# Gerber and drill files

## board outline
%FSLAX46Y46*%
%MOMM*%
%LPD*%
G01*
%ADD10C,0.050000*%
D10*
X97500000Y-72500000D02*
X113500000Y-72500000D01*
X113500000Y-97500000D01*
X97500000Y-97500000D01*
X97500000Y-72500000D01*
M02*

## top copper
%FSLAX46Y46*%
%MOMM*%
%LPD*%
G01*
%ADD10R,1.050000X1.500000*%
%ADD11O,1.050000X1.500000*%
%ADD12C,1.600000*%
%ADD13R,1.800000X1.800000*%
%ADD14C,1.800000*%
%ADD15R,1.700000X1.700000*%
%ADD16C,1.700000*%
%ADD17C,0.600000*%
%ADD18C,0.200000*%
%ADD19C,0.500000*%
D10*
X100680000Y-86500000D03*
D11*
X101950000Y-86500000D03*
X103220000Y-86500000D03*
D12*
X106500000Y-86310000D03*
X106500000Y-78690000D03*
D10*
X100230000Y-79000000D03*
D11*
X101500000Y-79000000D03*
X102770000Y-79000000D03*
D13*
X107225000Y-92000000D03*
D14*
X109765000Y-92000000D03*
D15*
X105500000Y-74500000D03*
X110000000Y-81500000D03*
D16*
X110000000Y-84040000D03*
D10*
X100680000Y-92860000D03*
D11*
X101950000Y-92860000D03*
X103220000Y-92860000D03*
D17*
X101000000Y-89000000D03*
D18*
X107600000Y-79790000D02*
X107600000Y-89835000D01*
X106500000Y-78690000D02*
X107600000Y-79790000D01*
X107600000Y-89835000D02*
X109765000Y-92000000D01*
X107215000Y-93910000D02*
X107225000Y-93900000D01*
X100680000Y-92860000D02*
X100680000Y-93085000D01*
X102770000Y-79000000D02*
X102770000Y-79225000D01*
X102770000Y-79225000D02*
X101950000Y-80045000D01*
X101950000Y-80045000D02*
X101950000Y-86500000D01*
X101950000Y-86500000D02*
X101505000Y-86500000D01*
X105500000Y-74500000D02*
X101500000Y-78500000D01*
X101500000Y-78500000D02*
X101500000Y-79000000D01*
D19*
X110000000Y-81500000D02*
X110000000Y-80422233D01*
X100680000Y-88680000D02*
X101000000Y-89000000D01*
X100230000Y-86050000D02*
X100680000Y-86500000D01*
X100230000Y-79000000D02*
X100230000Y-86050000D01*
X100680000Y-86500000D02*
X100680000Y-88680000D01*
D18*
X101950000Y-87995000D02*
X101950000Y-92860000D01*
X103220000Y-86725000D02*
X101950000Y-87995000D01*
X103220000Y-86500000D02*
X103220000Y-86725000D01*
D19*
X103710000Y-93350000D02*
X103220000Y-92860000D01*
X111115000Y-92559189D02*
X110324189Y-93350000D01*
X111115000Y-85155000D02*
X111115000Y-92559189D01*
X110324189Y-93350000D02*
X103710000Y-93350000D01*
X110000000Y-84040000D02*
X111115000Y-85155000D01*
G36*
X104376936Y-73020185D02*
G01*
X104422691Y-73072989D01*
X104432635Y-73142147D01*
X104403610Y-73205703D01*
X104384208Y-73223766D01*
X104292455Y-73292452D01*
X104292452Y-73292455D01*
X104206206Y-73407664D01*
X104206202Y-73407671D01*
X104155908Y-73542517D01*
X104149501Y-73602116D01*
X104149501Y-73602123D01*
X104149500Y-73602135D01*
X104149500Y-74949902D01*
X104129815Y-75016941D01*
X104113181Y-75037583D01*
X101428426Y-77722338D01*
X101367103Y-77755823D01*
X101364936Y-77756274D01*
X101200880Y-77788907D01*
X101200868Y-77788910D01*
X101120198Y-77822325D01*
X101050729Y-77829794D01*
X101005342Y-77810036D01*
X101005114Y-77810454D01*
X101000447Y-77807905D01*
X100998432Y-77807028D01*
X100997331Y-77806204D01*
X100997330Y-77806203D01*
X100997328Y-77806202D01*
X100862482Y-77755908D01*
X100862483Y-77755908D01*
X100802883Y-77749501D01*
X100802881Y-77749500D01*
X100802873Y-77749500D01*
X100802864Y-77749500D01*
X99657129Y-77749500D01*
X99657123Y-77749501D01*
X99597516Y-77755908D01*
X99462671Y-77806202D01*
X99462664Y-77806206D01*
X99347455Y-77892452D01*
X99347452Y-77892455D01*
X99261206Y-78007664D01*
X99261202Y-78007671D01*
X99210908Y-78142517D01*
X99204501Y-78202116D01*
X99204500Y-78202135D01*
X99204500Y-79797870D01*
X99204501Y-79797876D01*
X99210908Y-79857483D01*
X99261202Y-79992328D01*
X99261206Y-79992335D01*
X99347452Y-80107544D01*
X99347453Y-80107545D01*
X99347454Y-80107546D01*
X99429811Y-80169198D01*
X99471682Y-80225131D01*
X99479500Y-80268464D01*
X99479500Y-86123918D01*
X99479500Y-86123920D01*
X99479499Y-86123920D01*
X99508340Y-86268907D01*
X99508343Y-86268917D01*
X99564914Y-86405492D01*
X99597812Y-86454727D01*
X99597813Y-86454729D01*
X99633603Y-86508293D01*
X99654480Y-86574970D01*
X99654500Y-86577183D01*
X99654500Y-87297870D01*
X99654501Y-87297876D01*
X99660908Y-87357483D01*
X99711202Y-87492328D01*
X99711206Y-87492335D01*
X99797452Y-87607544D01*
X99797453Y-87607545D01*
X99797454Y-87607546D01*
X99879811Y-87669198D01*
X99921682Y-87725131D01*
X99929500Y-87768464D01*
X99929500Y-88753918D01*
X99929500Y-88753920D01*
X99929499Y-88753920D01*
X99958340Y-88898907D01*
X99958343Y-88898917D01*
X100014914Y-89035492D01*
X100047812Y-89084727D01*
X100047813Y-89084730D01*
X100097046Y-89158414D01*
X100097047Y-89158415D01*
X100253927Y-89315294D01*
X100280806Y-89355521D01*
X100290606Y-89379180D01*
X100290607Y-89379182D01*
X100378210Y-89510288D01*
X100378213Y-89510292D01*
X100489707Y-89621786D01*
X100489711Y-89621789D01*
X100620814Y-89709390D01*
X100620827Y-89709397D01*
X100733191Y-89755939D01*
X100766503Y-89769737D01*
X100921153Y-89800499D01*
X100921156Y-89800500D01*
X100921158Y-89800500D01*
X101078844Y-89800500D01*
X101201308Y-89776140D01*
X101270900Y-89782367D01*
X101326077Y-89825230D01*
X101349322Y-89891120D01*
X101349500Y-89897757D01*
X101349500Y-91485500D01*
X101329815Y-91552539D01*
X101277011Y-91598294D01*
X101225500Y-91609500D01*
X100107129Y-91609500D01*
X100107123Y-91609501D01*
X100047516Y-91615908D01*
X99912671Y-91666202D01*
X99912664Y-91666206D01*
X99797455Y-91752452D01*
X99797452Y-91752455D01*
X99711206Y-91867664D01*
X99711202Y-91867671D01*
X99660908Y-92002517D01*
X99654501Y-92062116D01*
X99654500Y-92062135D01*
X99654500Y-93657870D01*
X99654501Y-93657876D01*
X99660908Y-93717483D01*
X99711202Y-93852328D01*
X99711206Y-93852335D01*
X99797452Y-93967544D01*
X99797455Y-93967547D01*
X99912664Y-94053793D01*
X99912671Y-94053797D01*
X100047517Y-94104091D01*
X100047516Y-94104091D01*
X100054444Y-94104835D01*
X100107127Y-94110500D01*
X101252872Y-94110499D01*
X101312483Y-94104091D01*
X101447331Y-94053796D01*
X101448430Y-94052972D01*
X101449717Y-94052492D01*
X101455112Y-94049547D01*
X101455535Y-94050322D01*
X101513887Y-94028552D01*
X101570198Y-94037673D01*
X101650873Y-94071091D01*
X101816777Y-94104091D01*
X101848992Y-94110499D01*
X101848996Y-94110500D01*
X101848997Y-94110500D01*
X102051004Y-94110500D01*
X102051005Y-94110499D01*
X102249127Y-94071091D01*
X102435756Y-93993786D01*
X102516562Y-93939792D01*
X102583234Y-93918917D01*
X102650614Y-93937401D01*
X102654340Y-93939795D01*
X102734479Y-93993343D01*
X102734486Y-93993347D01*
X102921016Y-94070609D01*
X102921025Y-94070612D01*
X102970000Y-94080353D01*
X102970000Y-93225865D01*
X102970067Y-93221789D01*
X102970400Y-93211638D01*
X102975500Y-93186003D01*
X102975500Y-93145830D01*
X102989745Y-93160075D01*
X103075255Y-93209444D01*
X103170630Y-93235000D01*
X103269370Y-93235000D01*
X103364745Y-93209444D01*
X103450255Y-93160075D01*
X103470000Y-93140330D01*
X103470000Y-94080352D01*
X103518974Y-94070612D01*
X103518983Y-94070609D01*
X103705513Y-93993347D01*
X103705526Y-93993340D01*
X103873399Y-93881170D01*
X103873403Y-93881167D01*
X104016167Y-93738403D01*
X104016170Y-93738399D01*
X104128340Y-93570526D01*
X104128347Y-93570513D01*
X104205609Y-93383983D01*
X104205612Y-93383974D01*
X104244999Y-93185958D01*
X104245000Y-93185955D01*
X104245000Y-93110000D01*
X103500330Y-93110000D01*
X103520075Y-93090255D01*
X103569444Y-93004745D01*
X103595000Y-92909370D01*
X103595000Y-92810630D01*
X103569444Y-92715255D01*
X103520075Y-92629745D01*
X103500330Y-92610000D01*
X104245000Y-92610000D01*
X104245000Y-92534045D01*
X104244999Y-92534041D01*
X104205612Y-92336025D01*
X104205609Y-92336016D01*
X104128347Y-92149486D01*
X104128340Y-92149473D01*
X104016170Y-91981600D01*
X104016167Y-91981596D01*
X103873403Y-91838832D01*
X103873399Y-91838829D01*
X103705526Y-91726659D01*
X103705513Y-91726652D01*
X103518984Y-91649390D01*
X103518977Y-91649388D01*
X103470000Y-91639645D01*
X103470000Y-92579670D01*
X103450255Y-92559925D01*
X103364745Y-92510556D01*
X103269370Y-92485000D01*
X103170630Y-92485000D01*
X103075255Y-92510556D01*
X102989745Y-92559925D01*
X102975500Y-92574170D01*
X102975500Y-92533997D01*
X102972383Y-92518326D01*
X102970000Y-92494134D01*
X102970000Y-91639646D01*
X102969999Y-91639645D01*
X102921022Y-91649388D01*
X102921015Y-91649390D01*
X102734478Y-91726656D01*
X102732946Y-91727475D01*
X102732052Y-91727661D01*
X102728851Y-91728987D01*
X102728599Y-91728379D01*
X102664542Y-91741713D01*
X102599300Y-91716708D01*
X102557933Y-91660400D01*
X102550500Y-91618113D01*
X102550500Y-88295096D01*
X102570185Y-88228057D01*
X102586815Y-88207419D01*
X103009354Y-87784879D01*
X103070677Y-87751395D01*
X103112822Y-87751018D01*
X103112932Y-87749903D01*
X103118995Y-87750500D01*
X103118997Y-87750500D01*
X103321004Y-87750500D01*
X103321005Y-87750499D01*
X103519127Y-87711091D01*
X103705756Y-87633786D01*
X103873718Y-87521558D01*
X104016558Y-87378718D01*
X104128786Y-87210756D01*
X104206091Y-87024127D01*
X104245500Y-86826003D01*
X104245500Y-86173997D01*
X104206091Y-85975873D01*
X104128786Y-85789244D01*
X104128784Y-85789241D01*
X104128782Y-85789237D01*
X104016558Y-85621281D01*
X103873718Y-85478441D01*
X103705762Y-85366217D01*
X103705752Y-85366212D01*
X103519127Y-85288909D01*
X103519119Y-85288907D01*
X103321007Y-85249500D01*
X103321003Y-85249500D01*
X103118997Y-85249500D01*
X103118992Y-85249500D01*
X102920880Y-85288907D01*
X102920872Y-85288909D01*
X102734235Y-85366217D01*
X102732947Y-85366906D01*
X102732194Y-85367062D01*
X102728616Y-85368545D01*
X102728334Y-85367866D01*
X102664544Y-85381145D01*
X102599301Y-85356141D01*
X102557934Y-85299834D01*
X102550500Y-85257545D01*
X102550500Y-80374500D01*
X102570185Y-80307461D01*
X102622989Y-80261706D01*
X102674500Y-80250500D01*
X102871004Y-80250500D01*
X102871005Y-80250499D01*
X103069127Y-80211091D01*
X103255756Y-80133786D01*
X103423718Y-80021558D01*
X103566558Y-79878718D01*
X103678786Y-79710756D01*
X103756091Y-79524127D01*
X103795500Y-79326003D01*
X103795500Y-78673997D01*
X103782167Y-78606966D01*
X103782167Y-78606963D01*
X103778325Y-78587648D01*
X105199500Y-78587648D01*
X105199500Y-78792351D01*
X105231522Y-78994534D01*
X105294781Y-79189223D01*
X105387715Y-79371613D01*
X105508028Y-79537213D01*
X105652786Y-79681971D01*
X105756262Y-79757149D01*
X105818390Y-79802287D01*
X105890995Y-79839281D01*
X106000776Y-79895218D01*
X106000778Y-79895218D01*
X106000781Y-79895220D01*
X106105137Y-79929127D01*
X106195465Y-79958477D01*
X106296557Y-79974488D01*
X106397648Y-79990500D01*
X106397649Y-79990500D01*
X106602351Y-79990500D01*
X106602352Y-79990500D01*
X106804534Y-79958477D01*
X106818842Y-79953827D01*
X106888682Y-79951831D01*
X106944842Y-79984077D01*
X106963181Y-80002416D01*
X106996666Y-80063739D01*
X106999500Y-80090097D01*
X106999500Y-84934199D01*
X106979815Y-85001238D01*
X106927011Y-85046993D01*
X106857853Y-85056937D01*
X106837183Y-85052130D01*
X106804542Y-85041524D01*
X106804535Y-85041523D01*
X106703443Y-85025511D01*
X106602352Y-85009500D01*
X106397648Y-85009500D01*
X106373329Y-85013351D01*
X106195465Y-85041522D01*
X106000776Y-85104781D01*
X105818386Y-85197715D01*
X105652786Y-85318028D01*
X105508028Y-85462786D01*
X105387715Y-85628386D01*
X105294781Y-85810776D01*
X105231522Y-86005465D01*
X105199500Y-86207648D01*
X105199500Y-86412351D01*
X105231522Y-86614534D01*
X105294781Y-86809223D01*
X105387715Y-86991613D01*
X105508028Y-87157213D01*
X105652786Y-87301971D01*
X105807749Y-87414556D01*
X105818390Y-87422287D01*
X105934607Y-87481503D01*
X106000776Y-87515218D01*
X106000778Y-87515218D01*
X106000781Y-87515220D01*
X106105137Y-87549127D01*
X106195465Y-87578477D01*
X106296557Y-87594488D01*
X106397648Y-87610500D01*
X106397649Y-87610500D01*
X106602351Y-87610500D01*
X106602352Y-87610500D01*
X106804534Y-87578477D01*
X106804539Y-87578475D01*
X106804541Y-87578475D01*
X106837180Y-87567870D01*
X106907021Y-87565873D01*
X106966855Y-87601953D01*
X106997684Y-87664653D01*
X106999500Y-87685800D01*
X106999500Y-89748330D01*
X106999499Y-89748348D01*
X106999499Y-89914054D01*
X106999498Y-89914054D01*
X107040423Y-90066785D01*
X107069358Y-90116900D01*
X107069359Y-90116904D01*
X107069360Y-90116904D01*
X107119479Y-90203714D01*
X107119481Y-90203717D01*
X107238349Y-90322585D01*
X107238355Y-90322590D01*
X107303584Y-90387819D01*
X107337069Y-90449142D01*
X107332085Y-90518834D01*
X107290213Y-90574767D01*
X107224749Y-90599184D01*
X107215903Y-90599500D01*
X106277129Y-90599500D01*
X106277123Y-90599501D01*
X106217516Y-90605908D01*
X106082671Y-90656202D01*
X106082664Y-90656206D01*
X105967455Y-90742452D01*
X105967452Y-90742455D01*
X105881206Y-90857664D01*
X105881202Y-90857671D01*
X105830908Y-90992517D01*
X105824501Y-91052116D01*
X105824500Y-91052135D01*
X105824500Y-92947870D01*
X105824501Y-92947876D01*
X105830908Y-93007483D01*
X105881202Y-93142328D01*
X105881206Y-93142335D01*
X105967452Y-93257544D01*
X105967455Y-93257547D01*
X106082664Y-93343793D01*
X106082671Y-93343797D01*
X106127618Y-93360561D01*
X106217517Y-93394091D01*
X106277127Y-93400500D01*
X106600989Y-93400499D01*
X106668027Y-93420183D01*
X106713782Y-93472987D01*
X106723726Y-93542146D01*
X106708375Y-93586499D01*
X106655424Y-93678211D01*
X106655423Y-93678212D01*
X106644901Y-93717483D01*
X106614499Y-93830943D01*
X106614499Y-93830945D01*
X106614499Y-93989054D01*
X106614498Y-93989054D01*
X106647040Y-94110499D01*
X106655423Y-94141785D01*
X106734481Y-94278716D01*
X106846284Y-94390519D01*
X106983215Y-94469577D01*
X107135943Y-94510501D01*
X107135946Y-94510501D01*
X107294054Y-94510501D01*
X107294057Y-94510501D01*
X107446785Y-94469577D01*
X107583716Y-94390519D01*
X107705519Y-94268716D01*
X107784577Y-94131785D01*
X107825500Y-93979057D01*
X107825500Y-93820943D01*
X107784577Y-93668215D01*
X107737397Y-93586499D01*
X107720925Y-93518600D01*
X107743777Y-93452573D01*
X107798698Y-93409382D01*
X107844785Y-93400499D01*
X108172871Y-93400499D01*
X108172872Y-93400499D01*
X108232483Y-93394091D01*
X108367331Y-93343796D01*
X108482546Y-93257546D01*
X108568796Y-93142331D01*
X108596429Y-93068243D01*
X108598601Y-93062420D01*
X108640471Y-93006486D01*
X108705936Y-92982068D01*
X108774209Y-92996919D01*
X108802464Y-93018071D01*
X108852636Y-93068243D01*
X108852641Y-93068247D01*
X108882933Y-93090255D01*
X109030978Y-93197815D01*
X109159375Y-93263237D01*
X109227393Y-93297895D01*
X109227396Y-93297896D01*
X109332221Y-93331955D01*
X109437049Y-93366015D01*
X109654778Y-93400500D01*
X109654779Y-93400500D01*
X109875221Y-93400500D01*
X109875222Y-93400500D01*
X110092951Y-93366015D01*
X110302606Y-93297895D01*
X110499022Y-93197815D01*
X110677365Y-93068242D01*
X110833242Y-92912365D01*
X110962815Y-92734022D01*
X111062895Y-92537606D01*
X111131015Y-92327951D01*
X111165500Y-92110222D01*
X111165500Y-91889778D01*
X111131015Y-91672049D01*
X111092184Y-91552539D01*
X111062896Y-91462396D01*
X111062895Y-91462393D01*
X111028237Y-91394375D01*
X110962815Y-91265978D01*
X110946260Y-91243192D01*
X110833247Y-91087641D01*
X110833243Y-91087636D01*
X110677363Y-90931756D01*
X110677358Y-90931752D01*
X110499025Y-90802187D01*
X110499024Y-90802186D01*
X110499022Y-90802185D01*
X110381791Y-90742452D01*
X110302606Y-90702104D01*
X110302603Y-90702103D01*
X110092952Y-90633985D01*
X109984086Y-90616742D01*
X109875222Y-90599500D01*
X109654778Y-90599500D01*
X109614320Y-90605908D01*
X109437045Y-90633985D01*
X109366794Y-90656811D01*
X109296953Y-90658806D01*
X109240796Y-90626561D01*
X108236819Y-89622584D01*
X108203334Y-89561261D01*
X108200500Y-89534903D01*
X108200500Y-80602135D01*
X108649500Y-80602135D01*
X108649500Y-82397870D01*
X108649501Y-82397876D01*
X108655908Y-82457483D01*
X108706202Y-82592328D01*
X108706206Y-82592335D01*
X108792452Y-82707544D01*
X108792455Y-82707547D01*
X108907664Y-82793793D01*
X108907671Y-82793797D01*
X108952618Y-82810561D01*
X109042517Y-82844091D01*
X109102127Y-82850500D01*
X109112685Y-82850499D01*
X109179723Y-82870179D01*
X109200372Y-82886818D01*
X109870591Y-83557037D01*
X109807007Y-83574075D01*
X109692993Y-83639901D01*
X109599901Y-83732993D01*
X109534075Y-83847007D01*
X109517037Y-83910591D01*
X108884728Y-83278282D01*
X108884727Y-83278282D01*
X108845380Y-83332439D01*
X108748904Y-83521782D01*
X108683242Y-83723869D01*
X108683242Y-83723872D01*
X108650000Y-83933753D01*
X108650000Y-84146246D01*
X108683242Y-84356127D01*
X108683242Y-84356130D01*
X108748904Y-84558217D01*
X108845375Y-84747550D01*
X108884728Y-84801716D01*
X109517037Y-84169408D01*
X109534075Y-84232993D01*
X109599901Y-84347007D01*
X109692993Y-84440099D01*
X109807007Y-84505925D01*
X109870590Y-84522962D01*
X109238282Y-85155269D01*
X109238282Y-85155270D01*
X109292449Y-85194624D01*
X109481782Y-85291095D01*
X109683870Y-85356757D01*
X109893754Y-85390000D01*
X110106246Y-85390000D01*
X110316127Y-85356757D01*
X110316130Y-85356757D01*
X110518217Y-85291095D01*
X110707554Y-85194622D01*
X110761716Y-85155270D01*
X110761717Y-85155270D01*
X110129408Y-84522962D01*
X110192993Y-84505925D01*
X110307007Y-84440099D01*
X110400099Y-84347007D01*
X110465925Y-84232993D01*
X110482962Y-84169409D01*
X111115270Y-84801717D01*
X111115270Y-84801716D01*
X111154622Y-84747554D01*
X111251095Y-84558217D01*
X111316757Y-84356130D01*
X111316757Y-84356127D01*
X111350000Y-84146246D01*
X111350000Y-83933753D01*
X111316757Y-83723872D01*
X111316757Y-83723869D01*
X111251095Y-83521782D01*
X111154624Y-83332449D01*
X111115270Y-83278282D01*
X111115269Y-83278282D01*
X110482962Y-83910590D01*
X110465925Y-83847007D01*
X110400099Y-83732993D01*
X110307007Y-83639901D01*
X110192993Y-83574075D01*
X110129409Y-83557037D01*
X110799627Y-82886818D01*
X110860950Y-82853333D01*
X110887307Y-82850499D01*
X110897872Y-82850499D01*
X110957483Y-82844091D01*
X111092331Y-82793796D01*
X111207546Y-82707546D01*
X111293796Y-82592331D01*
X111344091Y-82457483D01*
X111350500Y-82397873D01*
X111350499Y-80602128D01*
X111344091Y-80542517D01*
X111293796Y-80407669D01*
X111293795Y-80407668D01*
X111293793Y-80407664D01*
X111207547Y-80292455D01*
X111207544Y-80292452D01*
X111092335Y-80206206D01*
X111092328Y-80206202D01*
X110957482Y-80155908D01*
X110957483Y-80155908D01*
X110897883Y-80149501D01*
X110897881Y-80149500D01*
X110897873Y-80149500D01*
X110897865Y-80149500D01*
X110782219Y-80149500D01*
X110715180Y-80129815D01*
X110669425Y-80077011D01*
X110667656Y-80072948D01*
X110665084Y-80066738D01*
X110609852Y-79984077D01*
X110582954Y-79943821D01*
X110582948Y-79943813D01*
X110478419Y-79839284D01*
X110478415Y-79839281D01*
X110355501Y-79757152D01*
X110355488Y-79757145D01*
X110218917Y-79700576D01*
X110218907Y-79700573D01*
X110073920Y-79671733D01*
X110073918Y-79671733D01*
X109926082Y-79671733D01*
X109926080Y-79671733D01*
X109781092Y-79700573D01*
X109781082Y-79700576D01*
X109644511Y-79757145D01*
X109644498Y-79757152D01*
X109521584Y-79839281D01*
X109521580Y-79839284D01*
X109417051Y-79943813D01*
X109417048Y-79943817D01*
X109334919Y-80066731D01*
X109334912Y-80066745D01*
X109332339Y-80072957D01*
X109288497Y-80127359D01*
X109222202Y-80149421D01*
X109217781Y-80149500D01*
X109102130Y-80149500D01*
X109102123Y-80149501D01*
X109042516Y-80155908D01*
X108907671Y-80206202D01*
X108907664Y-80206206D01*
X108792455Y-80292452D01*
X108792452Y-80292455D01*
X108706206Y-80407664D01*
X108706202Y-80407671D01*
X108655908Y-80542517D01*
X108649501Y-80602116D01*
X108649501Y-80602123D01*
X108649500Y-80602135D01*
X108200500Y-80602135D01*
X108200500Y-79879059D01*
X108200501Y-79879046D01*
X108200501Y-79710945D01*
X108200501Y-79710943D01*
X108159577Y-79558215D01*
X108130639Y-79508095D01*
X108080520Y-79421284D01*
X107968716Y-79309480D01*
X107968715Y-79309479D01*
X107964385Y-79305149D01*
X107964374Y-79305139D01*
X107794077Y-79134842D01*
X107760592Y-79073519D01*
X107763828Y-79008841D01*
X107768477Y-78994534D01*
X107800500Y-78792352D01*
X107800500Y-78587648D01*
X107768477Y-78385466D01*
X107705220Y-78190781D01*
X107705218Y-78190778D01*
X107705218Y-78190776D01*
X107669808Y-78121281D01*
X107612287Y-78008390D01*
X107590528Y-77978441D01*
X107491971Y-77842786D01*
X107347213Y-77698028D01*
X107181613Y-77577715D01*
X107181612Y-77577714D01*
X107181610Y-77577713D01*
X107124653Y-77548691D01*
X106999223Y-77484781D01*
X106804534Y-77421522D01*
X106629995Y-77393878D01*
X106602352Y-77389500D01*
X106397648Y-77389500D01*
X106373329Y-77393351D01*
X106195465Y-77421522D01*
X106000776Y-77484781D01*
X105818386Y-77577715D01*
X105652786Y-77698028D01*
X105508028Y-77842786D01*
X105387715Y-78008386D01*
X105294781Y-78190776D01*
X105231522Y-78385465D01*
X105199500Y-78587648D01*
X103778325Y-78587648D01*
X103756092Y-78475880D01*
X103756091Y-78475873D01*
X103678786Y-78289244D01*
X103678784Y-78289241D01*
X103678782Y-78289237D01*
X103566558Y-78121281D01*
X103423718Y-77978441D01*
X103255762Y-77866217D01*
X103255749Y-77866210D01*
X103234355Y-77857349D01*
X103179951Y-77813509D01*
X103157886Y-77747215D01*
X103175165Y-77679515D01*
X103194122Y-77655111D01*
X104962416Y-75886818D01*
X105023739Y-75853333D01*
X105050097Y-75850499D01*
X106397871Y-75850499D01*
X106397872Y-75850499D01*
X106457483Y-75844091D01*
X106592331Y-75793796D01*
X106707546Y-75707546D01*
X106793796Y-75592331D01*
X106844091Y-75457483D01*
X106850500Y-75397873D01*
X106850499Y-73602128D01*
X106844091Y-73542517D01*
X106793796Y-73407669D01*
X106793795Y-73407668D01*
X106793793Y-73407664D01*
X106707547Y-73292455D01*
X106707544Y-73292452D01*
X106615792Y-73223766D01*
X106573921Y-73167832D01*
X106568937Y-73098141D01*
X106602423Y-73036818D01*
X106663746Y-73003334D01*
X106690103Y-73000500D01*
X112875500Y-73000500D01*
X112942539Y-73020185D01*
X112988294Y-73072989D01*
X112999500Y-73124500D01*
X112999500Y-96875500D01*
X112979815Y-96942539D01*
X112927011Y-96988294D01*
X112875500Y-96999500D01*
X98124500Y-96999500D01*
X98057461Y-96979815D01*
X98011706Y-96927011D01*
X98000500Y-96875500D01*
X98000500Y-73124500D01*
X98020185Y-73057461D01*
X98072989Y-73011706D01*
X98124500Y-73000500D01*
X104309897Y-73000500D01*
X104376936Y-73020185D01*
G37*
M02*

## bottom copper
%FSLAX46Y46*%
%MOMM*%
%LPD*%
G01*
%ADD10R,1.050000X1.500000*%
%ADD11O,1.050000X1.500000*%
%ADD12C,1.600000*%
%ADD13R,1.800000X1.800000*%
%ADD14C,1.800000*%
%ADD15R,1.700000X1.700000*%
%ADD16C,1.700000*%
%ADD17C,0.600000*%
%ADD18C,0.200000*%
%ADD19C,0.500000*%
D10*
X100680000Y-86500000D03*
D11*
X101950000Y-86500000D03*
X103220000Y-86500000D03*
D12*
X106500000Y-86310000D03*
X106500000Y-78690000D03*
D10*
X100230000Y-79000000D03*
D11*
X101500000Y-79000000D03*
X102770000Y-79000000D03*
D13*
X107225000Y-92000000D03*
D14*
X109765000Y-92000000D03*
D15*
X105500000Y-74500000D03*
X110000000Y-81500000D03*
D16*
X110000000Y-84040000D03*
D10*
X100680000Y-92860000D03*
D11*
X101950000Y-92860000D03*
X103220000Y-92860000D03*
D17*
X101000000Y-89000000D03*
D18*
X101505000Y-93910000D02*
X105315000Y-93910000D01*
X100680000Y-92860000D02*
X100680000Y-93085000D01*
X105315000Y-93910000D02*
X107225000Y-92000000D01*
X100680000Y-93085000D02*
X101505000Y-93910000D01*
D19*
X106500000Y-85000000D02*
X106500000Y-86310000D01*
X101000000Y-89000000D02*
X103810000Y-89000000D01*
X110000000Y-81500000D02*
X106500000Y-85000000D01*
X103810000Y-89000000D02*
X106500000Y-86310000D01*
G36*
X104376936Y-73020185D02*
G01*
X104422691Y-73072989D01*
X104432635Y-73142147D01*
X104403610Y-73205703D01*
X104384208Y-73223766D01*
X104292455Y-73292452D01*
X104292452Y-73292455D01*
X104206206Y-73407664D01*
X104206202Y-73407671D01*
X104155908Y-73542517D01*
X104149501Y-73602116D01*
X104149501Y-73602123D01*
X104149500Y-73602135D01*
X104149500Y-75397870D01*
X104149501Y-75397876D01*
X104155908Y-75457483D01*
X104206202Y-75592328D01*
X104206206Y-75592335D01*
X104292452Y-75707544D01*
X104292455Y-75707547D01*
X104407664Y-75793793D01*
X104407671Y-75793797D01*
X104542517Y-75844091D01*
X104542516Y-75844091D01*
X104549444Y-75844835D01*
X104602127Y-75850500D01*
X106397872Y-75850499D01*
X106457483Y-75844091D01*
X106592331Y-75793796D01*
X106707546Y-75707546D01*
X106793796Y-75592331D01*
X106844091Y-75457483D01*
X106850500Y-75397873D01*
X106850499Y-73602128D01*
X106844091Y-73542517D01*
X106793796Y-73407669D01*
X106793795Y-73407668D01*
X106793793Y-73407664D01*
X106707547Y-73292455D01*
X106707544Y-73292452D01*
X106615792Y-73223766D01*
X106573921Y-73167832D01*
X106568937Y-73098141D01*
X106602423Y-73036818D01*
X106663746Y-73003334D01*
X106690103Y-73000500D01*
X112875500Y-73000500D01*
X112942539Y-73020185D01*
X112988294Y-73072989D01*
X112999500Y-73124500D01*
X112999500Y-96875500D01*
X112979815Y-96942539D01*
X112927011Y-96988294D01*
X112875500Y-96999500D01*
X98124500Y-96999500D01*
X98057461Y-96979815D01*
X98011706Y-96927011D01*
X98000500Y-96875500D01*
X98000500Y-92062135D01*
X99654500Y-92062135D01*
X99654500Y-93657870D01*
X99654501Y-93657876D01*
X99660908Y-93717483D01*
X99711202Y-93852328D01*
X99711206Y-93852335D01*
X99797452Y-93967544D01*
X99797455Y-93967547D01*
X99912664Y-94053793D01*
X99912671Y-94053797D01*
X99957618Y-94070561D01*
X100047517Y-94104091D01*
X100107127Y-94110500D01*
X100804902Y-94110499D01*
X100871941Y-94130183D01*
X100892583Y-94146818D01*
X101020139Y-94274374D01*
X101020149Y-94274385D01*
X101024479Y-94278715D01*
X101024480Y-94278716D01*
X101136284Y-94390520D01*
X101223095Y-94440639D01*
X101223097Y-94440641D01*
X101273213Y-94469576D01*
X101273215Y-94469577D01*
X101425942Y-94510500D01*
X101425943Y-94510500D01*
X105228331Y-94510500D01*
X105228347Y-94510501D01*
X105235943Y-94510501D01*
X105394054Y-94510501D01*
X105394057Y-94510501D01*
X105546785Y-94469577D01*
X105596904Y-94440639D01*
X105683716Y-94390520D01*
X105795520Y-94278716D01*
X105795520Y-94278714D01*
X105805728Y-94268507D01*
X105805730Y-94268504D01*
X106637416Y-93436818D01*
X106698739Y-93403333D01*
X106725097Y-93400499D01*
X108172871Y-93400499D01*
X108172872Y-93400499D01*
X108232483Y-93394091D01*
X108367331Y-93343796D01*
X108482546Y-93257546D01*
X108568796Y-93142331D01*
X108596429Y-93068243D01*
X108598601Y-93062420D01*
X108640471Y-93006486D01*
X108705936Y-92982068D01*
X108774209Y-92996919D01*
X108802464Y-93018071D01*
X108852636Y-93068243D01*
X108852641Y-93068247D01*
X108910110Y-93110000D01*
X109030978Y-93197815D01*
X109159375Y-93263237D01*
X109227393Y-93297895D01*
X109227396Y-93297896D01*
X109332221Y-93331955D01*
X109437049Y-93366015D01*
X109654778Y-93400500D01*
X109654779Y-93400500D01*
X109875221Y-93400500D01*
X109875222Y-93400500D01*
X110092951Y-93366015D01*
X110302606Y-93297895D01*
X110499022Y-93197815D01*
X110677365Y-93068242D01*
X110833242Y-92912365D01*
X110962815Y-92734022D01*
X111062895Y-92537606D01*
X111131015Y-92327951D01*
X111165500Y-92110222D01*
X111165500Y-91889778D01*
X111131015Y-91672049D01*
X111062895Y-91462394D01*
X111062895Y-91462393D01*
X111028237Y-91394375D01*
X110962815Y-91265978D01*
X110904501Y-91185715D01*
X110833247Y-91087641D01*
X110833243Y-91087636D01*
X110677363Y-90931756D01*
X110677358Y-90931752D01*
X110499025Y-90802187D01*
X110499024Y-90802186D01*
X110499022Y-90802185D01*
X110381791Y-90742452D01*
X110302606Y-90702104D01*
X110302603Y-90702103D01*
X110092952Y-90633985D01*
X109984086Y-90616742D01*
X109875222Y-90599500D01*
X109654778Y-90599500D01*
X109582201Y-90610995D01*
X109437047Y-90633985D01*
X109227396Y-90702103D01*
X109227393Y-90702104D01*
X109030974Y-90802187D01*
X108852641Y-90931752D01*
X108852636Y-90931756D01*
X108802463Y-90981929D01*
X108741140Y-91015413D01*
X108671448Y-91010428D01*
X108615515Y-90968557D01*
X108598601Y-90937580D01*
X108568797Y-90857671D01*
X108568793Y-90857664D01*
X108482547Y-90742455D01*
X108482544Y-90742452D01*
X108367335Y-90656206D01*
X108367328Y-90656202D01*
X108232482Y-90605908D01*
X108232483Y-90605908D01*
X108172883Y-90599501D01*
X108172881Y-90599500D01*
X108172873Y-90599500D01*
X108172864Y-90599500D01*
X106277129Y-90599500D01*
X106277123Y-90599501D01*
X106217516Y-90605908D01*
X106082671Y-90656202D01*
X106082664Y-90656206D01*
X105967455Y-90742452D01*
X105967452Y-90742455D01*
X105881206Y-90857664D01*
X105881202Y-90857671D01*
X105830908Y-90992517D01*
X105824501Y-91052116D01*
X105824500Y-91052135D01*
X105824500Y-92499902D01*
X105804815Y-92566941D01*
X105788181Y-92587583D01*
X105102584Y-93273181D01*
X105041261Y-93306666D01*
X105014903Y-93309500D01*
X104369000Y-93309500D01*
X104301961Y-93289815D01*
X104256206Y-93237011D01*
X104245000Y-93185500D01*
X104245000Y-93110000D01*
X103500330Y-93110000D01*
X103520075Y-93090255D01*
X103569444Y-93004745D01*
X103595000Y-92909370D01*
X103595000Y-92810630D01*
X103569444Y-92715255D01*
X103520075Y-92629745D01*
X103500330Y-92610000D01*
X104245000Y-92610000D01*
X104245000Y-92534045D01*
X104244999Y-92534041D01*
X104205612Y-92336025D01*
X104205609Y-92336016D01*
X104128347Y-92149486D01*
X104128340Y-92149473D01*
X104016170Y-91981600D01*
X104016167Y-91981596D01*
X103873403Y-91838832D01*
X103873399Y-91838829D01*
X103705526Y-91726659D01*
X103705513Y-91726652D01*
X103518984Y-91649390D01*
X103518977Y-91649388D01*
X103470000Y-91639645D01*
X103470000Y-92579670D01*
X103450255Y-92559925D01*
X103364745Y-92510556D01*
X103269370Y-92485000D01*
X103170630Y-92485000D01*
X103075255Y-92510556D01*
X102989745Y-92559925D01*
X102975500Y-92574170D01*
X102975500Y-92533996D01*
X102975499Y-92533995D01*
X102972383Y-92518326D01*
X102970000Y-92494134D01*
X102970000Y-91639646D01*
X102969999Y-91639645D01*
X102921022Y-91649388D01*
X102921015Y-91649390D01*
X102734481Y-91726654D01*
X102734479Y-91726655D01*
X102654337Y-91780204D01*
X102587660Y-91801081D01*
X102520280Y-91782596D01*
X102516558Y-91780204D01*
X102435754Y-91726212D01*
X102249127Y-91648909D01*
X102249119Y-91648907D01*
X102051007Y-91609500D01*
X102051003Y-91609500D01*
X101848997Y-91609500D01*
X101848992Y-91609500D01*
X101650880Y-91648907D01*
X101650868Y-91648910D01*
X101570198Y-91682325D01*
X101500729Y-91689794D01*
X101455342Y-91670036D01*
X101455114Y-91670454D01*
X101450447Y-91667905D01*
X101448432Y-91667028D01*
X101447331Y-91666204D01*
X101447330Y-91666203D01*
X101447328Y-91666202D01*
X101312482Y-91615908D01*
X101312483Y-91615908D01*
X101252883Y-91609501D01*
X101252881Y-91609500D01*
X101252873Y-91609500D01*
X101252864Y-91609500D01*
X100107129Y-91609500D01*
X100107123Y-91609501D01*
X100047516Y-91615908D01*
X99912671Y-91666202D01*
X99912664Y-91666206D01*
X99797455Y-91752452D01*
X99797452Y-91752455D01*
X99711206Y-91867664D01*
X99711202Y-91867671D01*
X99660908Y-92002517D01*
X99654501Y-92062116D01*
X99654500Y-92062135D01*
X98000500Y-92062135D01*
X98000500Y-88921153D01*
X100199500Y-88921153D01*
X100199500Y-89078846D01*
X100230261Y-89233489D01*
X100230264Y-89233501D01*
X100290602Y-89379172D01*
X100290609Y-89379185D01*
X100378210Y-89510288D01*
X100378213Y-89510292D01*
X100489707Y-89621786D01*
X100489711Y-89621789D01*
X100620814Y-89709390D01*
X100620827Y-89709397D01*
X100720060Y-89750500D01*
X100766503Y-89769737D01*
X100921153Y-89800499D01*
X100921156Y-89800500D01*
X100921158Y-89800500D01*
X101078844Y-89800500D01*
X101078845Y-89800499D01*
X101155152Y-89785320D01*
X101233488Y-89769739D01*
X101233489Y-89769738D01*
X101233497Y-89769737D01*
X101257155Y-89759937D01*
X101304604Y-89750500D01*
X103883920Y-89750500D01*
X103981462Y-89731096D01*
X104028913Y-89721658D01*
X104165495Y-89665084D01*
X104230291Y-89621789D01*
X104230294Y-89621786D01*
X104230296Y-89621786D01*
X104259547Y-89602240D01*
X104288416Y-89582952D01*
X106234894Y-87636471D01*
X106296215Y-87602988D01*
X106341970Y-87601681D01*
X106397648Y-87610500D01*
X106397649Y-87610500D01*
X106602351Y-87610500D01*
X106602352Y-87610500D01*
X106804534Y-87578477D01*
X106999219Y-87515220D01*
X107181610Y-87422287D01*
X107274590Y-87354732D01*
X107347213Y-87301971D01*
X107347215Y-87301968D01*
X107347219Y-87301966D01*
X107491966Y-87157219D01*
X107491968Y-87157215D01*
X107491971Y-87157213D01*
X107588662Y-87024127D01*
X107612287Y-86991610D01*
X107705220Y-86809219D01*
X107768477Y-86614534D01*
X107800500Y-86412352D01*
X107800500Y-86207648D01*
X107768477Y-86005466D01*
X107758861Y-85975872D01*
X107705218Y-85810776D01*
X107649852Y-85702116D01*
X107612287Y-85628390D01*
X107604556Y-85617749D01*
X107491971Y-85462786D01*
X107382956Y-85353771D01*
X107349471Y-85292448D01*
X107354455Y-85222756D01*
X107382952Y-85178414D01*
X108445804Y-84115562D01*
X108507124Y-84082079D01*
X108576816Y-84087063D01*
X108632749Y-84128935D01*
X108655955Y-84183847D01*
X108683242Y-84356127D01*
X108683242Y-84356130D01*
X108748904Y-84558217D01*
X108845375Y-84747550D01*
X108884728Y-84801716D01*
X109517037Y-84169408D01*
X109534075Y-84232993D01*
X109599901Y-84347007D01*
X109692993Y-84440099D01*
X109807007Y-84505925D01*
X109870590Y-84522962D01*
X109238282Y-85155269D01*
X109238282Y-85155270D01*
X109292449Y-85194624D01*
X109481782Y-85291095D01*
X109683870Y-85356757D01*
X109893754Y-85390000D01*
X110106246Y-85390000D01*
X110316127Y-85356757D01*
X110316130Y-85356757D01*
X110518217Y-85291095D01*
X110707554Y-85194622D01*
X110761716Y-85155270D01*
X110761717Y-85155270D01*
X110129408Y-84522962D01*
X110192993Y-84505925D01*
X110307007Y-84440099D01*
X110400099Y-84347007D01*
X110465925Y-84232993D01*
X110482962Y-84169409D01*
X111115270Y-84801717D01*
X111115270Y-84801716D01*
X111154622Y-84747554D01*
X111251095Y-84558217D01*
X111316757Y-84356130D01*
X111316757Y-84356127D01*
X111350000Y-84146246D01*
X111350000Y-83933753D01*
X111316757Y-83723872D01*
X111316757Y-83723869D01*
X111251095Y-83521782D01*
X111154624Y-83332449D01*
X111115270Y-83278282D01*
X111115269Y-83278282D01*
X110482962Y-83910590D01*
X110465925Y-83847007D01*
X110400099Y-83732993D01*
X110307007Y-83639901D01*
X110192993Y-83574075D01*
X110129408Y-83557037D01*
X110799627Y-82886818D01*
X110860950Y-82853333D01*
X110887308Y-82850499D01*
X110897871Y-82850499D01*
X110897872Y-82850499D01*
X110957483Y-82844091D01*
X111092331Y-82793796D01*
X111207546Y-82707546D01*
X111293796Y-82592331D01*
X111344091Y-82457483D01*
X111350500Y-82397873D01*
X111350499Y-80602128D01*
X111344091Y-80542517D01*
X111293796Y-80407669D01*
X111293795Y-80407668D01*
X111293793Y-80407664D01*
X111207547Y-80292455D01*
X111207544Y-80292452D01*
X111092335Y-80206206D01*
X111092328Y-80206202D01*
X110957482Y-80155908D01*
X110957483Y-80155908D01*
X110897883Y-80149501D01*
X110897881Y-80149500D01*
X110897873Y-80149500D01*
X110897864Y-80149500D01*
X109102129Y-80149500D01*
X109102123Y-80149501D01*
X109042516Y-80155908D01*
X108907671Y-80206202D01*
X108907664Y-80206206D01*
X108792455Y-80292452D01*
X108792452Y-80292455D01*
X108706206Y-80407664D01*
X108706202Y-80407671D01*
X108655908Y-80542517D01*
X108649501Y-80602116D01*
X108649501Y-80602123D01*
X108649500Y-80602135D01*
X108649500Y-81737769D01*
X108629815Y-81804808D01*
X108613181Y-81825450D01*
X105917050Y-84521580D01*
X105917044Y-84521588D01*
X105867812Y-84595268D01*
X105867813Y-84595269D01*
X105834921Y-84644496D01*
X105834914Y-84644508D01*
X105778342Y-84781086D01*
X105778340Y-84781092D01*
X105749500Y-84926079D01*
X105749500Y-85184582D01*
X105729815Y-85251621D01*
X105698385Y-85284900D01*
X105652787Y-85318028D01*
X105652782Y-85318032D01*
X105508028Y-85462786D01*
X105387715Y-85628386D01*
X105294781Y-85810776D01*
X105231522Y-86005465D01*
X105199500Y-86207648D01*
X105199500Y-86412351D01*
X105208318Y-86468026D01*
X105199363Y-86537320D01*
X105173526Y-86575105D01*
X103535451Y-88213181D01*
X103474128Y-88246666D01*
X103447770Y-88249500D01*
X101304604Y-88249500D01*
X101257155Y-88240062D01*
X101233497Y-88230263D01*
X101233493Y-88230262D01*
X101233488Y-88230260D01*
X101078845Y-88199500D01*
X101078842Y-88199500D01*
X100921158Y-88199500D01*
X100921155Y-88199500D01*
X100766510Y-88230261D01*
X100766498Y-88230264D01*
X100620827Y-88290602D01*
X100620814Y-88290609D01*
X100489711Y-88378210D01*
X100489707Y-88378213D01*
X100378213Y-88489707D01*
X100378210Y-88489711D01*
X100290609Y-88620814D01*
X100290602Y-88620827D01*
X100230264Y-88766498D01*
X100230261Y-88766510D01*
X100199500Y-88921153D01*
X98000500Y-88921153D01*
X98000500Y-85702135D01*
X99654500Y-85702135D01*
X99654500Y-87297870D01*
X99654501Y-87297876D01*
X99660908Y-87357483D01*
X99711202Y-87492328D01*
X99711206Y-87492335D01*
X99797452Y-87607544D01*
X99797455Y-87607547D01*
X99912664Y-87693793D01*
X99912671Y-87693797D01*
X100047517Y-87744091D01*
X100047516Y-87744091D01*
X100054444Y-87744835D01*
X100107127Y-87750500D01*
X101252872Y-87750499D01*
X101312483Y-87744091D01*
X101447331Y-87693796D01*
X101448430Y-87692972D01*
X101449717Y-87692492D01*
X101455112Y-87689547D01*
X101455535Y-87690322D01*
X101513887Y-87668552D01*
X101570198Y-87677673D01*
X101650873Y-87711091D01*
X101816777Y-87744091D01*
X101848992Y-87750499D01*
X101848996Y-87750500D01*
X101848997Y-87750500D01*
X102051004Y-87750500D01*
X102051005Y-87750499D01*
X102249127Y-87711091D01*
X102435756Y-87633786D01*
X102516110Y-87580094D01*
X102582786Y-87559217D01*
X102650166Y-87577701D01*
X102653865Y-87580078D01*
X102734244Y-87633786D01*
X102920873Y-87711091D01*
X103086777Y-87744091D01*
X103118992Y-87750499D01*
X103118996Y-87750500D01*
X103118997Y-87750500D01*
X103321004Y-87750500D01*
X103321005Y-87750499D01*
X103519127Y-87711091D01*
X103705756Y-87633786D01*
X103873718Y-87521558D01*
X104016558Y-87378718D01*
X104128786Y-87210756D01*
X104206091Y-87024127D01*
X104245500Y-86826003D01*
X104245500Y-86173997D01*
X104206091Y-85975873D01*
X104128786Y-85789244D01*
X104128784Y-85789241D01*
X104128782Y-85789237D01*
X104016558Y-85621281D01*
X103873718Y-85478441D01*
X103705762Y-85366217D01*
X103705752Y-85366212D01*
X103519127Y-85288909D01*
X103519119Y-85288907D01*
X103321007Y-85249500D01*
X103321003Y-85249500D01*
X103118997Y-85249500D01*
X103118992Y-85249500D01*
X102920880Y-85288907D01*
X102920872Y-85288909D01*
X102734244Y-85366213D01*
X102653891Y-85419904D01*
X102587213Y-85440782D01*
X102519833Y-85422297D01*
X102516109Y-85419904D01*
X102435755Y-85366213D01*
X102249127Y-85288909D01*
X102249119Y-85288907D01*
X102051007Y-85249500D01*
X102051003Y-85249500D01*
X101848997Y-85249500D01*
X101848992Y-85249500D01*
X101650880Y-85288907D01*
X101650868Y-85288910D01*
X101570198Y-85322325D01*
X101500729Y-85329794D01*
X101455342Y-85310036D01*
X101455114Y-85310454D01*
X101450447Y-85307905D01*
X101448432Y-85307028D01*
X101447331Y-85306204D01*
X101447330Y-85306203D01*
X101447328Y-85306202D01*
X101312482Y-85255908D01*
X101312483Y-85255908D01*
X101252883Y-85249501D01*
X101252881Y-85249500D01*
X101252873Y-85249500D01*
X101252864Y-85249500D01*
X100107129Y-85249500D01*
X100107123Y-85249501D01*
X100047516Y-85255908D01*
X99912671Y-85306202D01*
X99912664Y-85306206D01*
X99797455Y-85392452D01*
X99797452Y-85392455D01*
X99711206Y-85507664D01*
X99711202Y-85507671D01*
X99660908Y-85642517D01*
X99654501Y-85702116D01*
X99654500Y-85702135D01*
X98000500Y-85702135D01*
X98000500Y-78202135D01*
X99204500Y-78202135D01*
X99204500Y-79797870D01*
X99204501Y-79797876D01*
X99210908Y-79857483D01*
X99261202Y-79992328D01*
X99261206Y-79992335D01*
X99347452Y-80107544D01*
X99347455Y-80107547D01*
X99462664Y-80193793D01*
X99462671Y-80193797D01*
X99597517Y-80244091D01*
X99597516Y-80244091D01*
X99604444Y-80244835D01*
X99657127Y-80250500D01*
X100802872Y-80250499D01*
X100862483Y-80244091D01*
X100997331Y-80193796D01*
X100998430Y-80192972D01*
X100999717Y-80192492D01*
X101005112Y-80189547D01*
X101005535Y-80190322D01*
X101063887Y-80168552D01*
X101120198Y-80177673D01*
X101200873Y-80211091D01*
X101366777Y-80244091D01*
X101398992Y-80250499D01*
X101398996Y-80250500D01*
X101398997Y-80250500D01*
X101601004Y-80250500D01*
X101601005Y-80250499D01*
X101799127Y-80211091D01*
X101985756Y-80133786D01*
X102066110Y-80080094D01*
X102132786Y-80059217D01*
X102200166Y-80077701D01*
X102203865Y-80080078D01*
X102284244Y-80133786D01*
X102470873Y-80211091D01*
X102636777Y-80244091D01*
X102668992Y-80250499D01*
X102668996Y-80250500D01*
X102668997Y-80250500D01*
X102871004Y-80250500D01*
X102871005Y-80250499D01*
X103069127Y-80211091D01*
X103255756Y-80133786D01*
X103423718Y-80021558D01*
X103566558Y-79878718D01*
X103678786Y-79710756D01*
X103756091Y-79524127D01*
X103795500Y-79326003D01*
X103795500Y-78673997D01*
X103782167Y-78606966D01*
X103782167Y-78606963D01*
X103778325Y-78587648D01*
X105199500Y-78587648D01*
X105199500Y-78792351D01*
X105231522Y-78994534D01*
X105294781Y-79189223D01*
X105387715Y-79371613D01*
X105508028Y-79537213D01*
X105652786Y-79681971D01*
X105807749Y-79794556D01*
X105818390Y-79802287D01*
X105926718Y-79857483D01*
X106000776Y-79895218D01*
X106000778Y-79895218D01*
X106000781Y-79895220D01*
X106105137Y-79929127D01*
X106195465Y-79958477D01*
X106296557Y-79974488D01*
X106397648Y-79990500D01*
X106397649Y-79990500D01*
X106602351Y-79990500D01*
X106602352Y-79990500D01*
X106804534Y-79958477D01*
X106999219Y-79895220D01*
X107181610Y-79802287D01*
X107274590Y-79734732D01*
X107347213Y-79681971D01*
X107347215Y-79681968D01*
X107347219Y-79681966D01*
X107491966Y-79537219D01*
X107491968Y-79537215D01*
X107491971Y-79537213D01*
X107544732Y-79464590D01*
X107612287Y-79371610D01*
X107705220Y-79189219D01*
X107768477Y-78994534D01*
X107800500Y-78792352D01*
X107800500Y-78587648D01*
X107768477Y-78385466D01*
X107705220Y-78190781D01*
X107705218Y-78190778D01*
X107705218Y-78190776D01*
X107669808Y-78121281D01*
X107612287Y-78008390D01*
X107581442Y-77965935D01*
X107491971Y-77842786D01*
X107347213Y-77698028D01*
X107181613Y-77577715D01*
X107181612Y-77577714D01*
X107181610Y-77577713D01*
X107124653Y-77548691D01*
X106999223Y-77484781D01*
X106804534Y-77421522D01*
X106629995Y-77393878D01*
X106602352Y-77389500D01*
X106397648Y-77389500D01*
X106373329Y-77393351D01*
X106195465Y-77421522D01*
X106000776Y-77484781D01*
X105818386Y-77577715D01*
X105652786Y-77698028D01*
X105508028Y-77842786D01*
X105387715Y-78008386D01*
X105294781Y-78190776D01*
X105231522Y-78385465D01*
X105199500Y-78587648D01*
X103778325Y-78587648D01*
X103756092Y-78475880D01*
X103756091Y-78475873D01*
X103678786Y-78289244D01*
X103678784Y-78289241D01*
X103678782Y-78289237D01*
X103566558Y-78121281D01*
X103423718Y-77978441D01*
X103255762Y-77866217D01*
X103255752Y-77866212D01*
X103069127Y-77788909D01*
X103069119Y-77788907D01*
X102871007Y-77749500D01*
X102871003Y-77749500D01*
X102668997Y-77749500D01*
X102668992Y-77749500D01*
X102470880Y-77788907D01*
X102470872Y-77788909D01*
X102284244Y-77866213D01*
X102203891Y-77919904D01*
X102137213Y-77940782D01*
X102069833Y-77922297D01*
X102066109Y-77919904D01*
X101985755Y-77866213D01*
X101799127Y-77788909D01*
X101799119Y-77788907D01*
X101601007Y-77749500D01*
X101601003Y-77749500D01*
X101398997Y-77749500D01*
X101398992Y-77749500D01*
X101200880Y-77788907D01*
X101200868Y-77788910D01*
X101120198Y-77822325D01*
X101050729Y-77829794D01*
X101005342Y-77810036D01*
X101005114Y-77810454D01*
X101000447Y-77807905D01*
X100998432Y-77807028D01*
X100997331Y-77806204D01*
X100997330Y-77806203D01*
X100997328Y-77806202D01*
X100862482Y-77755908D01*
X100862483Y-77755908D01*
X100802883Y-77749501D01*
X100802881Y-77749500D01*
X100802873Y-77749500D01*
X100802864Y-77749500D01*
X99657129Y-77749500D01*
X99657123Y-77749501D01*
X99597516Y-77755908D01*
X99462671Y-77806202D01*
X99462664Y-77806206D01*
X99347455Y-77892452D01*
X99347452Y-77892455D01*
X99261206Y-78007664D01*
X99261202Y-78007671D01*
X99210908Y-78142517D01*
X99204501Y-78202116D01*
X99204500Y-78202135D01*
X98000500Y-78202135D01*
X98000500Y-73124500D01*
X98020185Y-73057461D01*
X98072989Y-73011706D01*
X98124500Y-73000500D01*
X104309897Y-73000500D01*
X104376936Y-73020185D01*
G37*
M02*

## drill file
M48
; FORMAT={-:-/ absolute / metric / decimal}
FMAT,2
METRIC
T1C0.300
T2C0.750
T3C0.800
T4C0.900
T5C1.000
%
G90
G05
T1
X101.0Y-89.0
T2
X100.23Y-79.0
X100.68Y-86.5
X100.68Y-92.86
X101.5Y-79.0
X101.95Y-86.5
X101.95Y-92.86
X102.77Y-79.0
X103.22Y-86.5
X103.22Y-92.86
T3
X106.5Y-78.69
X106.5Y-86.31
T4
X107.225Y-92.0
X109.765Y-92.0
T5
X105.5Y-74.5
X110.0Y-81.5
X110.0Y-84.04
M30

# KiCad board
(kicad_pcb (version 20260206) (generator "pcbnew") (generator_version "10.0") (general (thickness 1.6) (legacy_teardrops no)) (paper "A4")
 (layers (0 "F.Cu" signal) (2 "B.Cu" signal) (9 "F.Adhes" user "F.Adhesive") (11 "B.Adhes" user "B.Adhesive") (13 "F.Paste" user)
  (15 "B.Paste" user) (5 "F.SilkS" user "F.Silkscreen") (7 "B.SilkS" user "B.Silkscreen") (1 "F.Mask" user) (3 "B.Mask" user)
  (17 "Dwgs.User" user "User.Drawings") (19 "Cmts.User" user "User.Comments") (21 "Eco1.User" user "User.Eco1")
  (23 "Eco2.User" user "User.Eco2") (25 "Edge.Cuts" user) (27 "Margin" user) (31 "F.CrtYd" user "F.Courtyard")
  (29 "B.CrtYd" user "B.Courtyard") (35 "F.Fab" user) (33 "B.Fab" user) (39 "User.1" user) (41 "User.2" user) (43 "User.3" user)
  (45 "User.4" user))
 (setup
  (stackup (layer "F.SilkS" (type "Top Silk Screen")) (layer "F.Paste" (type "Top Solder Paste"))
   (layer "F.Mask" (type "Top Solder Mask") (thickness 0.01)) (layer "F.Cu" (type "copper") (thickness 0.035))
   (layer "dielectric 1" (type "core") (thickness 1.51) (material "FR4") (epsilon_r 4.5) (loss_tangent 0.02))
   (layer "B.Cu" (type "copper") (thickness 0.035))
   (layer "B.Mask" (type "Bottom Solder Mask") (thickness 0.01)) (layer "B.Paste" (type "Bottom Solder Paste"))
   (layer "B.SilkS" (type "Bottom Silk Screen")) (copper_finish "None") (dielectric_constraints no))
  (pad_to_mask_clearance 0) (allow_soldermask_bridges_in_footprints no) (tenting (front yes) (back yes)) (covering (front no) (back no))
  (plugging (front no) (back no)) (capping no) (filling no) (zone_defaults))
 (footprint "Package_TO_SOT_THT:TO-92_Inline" (layer "F.Cu") (at 100.68 86.5)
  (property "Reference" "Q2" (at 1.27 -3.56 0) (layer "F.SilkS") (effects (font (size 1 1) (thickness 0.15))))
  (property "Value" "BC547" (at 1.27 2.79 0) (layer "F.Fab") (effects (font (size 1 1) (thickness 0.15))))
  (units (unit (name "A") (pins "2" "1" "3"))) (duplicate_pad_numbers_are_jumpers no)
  (pad "1" thru_hole rect (at 0 0) (size 1.05 1.5) (drill 0.75) (layers "*.Cu" "*.Mask") (remove_unused_layers no) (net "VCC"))
  (pad "2" thru_hole oval (at 1.27 0) (size 1.05 1.5) (drill 0.75) (layers "*.Cu" "*.Mask") (remove_unused_layers no) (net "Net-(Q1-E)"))
  (pad "3" thru_hole oval (at 2.54 0) (size 1.05 1.5) (drill 0.75) (layers "*.Cu" "*.Mask") (remove_unused_layers no) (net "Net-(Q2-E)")))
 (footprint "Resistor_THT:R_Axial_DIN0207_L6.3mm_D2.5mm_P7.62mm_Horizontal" (layer "F.Cu") (at 106.5 86.31 90)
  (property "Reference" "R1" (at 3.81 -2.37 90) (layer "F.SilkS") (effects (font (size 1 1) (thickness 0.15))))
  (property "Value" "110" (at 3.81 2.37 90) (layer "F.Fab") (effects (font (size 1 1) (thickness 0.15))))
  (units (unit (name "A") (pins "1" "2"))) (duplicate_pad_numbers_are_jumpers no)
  (pad "1" thru_hole circle (at 0 0 90) (size 1.6 1.6) (drill 0.8) (layers "*.Cu" "*.Mask") (remove_unused_layers no) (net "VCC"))
  (pad "2" thru_hole circle (at 7.62 0 90) (size 1.6 1.6) (drill 0.8) (layers "*.Cu" "*.Mask") (remove_unused_layers no) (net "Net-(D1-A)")))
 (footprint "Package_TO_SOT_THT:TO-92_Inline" (layer "F.Cu") (at 100.23 79)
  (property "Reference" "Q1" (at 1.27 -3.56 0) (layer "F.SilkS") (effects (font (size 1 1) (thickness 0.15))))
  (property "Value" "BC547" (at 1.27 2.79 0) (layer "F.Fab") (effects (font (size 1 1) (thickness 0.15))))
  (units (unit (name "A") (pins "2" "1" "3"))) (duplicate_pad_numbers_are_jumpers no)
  (pad "1" thru_hole rect (at 0 0) (size 1.05 1.5) (drill 0.75) (layers "*.Cu" "*.Mask") (remove_unused_layers no) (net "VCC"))
  (pad "2" thru_hole oval (at 1.27 0) (size 1.05 1.5) (drill 0.75) (layers "*.Cu" "*.Mask") (remove_unused_layers no) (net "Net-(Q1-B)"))
  (pad "3" thru_hole oval (at 2.54 0) (size 1.05 1.5) (drill 0.75) (layers "*.Cu" "*.Mask") (remove_unused_layers no) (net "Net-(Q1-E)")))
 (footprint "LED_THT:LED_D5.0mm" (layer "F.Cu") (at 107.225 92)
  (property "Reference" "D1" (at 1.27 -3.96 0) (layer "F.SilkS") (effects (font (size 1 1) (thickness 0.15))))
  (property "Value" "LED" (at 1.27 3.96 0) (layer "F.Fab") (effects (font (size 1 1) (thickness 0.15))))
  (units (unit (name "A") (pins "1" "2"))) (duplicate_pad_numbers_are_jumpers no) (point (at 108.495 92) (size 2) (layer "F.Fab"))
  (pad "1" thru_hole rect (at 0 0) (size 1.8 1.8) (drill 0.9) (layers "*.Cu" "*.Mask") (remove_unused_layers no) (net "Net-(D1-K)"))
  (pad "2" thru_hole circle (at 2.54 0) (size 1.8 1.8) (drill 0.9) (layers "*.Cu" "*.Mask") (remove_unused_layers no) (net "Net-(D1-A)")))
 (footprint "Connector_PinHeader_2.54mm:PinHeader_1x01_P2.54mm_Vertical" (layer "F.Cu") (at 105.5 74.5)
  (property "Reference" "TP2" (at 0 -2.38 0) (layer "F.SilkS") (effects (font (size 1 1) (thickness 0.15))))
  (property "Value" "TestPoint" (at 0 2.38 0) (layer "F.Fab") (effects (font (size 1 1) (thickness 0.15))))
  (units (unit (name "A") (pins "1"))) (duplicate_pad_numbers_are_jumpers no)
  (pad "1" thru_hole rect (at 0 0) (size 1.7 1.7) (drill 1) (layers "*.Cu" "*.Mask") (remove_unused_layers no) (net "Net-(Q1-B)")))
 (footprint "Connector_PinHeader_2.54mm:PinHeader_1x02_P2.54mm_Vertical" (layer "F.Cu") (at 110 81.5)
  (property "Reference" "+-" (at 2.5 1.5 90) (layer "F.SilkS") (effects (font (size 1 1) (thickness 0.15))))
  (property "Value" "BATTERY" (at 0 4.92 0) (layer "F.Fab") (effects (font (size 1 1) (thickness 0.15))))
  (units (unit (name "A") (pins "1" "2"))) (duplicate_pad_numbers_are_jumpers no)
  (pad "1" thru_hole rect (at 0 0) (size 1.7 1.7) (drill 1) (layers "*.Cu" "*.Mask") (remove_unused_layers no) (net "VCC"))
  (pad "2" thru_hole circle (at 0 2.54) (size 1.7 1.7) (drill 1) (layers "*.Cu" "*.Mask") (remove_unused_layers no) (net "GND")))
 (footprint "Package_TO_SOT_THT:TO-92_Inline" (layer "F.Cu") (at 100.68 92.86)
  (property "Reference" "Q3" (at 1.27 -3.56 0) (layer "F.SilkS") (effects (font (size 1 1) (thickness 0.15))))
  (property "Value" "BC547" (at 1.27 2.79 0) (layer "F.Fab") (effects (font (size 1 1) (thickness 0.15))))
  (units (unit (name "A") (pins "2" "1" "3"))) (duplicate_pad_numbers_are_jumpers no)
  (pad "1" thru_hole rect (at 0 0) (size 1.05 1.5) (drill 0.75) (layers "*.Cu" "*.Mask") (remove_unused_layers no) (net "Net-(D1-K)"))
  (pad "2" thru_hole oval (at 1.27 0) (size 1.05 1.5) (drill 0.75) (layers "*.Cu" "*.Mask") (remove_unused_layers no) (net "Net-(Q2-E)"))
  (pad "3" thru_hole oval (at 2.54 0) (size 1.05 1.5) (drill 0.75) (layers "*.Cu" "*.Mask") (remove_unused_layers no) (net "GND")))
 (gr_rect (start 97.5 72.5) (end 113.5 97.5) (stroke (width 0.05) (type default)) (fill no) (layer "Edge.Cuts"))
 (segment (start 107.6 79.79) (end 107.6 89.835) (width 0.2) (layer "F.Cu") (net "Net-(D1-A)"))
 (segment (start 106.5 78.69) (end 107.6 79.79) (width 0.2) (layer "F.Cu") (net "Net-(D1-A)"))
 (segment (start 107.6 89.835) (end 109.765 92) (width 0.2) (layer "F.Cu") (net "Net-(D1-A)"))
 (segment (start 107.215 93.91) (end 107.225 93.9) (width 0.2) (layer "F.Cu") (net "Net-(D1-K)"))
 (segment (start 100.68 92.86) (end 100.68 93.085) (width 0.2) (layer "F.Cu") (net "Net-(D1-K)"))
 (segment (start 101.505 93.91) (end 105.315 93.91) (width 0.2) (layer "B.Cu") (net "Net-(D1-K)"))
 (segment (start 100.68 92.86) (end 100.68 93.085) (width 0.2) (layer "B.Cu") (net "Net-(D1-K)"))
 (segment (start 105.315 93.91) (end 107.225 92) (width 0.2) (layer "B.Cu") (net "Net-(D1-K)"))
 (segment (start 100.68 93.085) (end 101.505 93.91) (width 0.2) (layer "B.Cu") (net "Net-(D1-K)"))
 (segment (start 102.77 79) (end 102.77 79.225) (width 0.2) (layer "F.Cu") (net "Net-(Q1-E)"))
 (segment (start 102.77 79.225) (end 101.95 80.045) (width 0.2) (layer "F.Cu") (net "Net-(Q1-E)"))
 (segment (start 101.95 80.045) (end 101.95 86.5) (width 0.2) (layer "F.Cu") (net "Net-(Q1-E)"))
 (segment (start 101.95 86.5) (end 101.505 86.5) (width 0.2) (layer "F.Cu") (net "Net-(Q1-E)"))
 (segment (start 105.5 74.5) (end 101.5 78.5) (width 0.2) (layer "F.Cu") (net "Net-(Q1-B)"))
 (segment (start 101.5 78.5) (end 101.5 79) (width 0.2) (layer "F.Cu") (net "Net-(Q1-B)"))
 (segment (start 110 81.5) (end 110 80.422233) (width 0.5) (layer "F.Cu") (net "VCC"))
 (segment (start 100.68 88.68) (end 101 89) (width 0.5) (layer "F.Cu") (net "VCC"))
 (segment (start 100.23 86.05) (end 100.68 86.5) (width 0.5) (layer "F.Cu") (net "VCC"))
 (segment (start 100.23 79) (end 100.23 86.05) (width 0.5) (layer "F.Cu") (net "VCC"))
 (segment (start 100.68 86.5) (end 100.68 88.68) (width 0.5) (layer "F.Cu") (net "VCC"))
 (via (at 101 89) (size 0.6) (drill 0.3) (layers "F.Cu" "B.Cu") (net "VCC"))
 (segment (start 106.5 85) (end 106.5 86.31) (width 0.5) (layer "B.Cu") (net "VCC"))
 (segment (start 101 89) (end 103.81 89) (width 0.5) (layer "B.Cu") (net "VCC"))
 (segment (start 110 81.5) (end 106.5 85) (width 0.5) (layer "B.Cu") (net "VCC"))
 (segment (start 103.81 89) (end 106.5 86.31) (width 0.5) (layer "B.Cu") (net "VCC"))
 (segment (start 101.95 87.995) (end 101.95 92.86) (width 0.2) (layer "F.Cu") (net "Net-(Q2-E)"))
 (segment (start 103.22 86.725) (end 101.95 87.995) (width 0.2) (layer "F.Cu") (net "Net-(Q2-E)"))
 (segment (start 103.22 86.5) (end 103.22 86.725) (width 0.2) (layer "F.Cu") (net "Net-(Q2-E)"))
 (segment (start 103.71 93.35) (end 103.22 92.86) (width 0.5) (layer "F.Cu") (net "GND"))
 (segment (start 111.115 92.559189) (end 110.324189 93.35) (width 0.5) (layer "F.Cu") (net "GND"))
 (segment (start 111.115 85.155) (end 111.115 92.559189) (width 0.5) (layer "F.Cu") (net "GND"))
 (segment (start 110.324189 93.35) (end 103.71 93.35) (width 0.5) (layer "F.Cu") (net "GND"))
 (segment (start 110 84.04) (end 111.115 85.155) (width 0.5) (layer "F.Cu") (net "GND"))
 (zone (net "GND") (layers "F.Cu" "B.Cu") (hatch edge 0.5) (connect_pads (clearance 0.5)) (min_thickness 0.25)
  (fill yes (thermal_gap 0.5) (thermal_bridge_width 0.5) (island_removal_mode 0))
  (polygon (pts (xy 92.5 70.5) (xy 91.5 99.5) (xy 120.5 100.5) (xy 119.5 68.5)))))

